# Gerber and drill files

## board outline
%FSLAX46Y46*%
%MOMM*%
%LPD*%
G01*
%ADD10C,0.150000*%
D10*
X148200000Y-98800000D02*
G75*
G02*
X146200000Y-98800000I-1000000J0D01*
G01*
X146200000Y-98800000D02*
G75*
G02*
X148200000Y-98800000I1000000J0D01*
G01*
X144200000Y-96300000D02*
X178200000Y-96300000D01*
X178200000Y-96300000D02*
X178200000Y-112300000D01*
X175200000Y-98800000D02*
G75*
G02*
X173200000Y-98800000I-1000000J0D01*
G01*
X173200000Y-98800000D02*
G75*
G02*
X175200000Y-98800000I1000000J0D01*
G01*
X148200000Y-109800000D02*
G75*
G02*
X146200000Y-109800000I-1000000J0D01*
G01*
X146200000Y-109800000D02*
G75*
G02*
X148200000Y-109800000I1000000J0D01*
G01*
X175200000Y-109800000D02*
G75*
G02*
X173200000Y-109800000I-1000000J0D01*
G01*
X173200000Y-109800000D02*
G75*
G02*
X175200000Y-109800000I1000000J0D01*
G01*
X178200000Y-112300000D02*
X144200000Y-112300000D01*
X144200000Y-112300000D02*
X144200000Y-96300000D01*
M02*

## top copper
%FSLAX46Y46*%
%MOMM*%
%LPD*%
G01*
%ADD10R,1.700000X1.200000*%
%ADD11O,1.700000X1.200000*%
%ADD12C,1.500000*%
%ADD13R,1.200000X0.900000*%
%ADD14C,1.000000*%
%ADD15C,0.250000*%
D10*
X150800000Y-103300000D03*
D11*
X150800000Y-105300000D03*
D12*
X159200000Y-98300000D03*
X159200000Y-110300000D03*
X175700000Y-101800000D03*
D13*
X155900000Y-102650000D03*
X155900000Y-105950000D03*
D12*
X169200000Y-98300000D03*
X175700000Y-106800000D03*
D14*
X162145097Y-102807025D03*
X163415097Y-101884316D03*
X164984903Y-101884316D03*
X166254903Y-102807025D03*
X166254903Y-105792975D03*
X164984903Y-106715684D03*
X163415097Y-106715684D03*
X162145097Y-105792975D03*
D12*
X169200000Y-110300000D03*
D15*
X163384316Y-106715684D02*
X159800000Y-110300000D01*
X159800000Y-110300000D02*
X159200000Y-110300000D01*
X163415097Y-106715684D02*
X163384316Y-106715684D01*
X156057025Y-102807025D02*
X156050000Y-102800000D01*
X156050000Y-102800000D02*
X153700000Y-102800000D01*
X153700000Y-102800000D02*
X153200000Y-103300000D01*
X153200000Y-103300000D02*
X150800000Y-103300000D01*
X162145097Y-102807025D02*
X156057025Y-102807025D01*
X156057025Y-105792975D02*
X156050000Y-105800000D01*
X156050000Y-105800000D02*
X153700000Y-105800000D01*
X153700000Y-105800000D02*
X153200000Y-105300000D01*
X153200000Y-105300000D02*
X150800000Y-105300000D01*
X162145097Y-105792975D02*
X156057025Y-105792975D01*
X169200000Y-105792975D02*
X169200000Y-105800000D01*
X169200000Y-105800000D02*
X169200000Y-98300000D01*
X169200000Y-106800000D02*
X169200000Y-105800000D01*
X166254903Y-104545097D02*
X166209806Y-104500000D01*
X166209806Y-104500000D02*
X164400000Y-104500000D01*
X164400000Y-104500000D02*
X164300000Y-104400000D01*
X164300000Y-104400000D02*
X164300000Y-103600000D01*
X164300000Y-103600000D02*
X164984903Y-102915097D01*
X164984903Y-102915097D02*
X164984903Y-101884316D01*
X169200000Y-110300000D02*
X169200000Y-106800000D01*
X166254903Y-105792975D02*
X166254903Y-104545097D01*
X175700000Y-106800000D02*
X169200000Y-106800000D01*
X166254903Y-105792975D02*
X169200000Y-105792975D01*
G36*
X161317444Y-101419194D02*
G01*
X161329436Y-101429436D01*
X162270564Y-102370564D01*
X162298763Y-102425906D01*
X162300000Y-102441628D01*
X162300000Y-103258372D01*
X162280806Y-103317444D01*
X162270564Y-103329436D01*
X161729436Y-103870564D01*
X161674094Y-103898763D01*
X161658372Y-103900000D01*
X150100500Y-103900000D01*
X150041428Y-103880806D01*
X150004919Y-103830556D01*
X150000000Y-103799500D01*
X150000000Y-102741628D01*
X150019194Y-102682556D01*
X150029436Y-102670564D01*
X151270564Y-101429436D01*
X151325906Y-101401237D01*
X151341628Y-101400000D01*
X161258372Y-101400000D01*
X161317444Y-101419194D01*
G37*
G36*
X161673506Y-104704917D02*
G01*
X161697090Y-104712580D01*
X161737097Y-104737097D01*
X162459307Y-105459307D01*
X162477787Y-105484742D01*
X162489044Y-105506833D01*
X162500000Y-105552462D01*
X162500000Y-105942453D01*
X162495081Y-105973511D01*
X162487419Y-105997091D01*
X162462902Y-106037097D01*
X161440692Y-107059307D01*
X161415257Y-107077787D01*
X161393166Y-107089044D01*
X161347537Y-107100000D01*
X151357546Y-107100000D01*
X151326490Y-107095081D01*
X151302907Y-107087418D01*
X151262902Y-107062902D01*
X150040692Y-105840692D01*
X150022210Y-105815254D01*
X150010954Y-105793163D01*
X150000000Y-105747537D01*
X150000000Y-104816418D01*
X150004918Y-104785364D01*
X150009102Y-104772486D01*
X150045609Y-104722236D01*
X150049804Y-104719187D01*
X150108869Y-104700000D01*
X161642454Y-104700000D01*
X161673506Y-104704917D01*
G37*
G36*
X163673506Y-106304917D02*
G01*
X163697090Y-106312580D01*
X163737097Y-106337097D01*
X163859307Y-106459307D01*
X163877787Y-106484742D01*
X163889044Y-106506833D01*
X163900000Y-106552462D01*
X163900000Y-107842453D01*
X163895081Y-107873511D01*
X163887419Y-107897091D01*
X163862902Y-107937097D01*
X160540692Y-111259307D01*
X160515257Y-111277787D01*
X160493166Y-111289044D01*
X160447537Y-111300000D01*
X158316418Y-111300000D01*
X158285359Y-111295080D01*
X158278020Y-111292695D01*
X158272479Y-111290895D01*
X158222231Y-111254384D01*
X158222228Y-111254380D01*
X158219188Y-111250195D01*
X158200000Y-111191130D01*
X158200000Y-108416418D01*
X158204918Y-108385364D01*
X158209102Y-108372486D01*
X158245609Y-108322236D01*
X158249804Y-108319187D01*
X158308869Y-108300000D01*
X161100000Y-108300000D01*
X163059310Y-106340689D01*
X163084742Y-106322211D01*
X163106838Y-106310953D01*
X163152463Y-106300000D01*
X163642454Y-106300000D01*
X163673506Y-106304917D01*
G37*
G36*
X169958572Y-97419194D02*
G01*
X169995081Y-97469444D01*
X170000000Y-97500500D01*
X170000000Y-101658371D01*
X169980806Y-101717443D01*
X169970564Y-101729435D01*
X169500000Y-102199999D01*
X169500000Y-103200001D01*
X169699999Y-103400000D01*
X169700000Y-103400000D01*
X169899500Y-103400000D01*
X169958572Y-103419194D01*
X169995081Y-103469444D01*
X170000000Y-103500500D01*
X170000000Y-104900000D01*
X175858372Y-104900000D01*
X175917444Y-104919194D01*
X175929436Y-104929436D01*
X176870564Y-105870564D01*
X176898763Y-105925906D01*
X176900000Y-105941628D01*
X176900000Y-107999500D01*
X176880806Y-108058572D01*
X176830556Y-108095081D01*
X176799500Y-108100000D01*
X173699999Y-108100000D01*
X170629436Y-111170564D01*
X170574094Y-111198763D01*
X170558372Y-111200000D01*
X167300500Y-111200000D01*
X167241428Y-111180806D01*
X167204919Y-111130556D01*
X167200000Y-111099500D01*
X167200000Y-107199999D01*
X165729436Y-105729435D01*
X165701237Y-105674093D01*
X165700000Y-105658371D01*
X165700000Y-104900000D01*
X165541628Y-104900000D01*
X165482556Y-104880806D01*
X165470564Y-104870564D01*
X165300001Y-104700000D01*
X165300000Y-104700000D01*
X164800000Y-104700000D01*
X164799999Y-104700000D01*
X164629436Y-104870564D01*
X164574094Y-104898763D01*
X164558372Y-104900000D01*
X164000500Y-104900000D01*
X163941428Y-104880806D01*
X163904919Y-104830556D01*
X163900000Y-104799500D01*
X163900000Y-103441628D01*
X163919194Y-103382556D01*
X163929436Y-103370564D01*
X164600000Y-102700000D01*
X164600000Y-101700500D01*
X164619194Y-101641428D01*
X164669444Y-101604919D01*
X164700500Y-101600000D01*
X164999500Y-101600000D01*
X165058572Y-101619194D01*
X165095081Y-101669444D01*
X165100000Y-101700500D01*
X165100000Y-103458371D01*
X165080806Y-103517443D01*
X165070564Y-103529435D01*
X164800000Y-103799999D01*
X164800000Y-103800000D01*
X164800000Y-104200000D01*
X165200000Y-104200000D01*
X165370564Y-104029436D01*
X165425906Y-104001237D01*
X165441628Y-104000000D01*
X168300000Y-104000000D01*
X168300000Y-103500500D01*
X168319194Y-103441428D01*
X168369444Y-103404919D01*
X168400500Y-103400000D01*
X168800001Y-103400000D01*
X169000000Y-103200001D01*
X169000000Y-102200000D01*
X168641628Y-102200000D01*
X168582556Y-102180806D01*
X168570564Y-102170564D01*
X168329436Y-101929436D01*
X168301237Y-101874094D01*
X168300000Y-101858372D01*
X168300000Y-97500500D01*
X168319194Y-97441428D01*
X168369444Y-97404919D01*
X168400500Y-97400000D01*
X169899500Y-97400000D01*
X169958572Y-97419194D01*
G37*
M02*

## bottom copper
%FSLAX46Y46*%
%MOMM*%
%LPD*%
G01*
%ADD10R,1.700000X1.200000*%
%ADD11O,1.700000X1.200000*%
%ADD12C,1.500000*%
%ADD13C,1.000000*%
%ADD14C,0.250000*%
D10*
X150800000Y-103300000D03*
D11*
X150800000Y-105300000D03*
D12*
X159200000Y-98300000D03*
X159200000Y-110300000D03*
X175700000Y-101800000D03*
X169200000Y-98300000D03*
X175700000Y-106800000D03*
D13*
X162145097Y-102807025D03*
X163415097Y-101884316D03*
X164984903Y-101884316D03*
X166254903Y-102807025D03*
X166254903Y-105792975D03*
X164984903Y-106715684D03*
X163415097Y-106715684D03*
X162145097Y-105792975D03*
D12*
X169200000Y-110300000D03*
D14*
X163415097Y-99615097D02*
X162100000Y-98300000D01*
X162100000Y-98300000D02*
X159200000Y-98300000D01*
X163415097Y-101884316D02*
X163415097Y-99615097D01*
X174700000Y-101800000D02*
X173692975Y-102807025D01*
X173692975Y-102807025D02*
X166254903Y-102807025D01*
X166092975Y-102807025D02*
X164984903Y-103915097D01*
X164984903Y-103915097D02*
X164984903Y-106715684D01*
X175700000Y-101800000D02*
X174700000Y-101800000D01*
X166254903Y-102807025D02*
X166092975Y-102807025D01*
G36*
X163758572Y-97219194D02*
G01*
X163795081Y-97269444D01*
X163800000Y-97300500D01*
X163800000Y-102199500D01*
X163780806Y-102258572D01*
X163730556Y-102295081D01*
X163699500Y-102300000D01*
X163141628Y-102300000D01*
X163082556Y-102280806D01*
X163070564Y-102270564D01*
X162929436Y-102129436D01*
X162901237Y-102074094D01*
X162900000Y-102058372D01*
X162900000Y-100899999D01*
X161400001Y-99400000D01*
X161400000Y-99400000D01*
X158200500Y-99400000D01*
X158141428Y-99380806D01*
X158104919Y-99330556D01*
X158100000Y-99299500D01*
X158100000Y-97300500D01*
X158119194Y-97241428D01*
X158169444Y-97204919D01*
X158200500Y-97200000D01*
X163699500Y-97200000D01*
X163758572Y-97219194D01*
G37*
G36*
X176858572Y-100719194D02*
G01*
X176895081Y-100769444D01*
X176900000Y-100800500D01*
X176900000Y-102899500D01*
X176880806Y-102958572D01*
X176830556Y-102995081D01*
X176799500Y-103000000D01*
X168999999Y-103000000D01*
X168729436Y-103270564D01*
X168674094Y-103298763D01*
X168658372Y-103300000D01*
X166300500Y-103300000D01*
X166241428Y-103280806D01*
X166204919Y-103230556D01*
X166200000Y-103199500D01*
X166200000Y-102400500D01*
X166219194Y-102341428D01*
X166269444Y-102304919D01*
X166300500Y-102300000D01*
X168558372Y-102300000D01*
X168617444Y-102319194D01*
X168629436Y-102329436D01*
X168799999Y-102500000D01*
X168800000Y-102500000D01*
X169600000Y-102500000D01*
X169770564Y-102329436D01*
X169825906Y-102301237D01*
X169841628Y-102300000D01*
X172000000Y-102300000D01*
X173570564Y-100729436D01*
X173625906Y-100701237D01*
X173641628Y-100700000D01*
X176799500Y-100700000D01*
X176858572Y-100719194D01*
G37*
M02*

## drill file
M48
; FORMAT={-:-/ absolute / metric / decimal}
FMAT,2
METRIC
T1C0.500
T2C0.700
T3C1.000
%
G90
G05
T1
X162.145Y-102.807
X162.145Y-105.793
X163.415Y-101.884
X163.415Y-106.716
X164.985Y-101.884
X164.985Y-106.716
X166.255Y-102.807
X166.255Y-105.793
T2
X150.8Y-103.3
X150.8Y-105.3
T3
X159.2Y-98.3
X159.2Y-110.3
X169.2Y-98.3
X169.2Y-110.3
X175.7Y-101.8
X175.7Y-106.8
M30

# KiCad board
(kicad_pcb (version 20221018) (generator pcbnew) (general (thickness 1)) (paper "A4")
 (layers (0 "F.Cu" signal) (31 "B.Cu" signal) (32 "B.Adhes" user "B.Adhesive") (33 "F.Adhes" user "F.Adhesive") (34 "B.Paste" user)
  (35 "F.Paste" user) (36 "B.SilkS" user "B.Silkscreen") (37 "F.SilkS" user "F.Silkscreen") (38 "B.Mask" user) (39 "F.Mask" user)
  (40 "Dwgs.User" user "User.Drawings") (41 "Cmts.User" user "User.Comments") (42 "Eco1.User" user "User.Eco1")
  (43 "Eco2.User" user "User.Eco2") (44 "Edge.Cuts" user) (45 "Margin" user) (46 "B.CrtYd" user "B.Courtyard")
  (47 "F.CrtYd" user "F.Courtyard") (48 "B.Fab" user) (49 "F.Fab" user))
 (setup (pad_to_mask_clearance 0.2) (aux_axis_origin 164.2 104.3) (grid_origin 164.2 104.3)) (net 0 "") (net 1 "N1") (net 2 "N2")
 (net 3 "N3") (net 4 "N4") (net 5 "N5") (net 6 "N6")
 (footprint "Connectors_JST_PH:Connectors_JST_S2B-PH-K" (layer "F.Cu") (at 150.8 103.3 -90)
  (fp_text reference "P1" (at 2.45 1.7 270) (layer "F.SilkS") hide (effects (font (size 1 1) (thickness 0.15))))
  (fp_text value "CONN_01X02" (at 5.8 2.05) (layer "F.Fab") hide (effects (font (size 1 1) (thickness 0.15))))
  (pad "1" thru_hole rect (at 0 0 270) (size 1.2 1.7) (drill 0.7) (layers "*.Cu" "*.Mask" "F.SilkS") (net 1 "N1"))
  (pad "2" thru_hole oval (at 2 0 270) (size 1.2 1.7) (drill 0.7) (layers "*.Cu" "*.Mask" "F.SilkS") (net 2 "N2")))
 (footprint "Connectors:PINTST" (layer "F.Cu") (at 159.2 98.3)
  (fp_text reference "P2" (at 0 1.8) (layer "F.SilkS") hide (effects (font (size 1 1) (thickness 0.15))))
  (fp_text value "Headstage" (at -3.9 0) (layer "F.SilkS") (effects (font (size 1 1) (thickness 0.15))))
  (pad "1" thru_hole circle (at 0 0) (size 1.5 1.5) (drill 1) (layers "*.Cu" "*.Mask") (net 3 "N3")))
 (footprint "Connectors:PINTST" (layer "F.Cu") (at 159.2 110.3)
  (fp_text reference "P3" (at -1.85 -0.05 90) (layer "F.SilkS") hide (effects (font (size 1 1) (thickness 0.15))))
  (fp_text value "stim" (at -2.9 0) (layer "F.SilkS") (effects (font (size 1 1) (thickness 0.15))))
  (pad "1" thru_hole circle (at 0 0) (size 1.5 1.5) (drill 1) (layers "*.Cu" "*.Mask") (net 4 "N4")))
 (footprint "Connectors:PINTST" (layer "F.Cu") (at 175.7 101.8)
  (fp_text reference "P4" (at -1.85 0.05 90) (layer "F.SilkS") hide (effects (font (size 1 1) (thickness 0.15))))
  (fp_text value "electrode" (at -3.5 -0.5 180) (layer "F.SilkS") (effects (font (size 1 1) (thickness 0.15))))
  (pad "1" thru_hole circle (at 0 0) (size 1.5 1.5) (drill 1) (layers "*.Cu" "*.Mask") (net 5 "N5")))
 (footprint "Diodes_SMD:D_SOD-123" (layer "F.Cu") (at 155.9 104.3 -90)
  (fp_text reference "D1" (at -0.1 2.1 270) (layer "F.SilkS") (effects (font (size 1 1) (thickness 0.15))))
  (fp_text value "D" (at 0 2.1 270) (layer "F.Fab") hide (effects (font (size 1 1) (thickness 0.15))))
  (pad "1" smd rect (at -1.65 0 270) (size 0.9 1.2) (layers "F.Cu" "F.Paste" "F.Mask") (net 1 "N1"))
  (pad "2" smd rect (at 1.65 0 270) (size 0.9 1.2) (layers "F.Cu" "F.Paste" "F.Mask") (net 2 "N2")))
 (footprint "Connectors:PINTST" (layer "F.Cu") (at 169.2 98.3)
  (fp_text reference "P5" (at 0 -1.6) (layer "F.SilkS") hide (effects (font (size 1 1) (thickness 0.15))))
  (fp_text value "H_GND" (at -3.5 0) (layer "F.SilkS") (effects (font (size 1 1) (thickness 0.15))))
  (pad "1" thru_hole circle (at 0 0) (size 1.5 1.5) (drill 1) (layers "*.Cu" "*.Mask") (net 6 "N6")))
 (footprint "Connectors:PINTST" (layer "F.Cu") (at 175.7 106.8)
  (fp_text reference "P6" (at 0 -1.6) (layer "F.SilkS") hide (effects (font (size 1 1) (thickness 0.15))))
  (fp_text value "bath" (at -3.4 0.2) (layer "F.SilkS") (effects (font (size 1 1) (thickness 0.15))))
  (pad "1" thru_hole circle (at 0 0) (size 1.5 1.5) (drill 1) (layers "*.Cu" "*.Mask") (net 6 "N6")))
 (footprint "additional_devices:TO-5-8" (layer "F.Cu") (at 164.2 104.3 90)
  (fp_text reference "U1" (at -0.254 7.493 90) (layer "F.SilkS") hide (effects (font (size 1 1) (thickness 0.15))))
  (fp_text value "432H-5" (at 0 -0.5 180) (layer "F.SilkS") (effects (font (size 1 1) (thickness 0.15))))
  (pad "1" thru_hole circle (at 1.492975 -2.054903 90) (size 1 1) (drill 0.5) (layers "*.Cu" "*.Mask") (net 1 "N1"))
  (pad "2" thru_hole circle (at 2.415684 -0.784903 54) (size 1 1) (drill 0.5) (layers "*.Cu" "*.Mask") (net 3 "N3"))
  (pad "3" thru_hole circle (at 2.415684 0.784903 18) (size 1 1) (drill 0.5) (layers "*.Cu" "*.Mask") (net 6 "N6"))
  (pad "4" thru_hole circle (at 1.492975 2.054903 342) (size 1 1) (drill 0.5) (layers "*.Cu" "*.Mask") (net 5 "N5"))
  (pad "5" thru_hole circle (at -1.492975 2.054903 270) (size 1 1) (drill 0.5) (layers "*.Cu" "*.Mask") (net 6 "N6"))
  (pad "6" thru_hole circle (at -2.415684 0.784903 234) (size 1 1) (drill 0.5) (layers "*.Cu" "*.Mask") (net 5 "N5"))
  (pad "7" thru_hole circle (at -2.415684 -0.784903 198) (size 1 1) (drill 0.5) (layers "*.Cu" "*.Mask") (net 4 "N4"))
  (pad "8" thru_hole circle (at -1.492975 -2.054903 162) (size 1 1) (drill 0.5) (layers "*.Cu" "*.Mask") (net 2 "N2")))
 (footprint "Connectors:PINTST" (layer "F.Cu") (at 169.2 110.3)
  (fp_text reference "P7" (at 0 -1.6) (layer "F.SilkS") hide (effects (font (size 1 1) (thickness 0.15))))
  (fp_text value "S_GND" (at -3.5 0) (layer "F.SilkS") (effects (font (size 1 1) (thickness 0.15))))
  (pad "1" thru_hole circle (at 0 0) (size 1.5 1.5) (drill 1) (layers "*.Cu" "*.Mask") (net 6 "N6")))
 (gr_circle (center 147.2 98.8) (end 148.2 98.8) (stroke (width 0.15) (type solid)) (fill none) (layer "Edge.Cuts"))
 (gr_line (start 144.2 96.3) (end 178.2 96.3) (stroke (width 0.15) (type solid)) (layer "Edge.Cuts"))
 (gr_line (start 178.2 96.3) (end 178.2 112.3) (stroke (width 0.15) (type solid)) (layer "Edge.Cuts"))
 (gr_circle (center 174.2 98.8) (end 175.2 98.8) (stroke (width 0.15) (type solid)) (fill none) (layer "Edge.Cuts"))
 (gr_circle (center 147.2 109.8) (end 148.2 109.8) (stroke (width 0.15) (type solid)) (fill none) (layer "Edge.Cuts"))
 (gr_circle (center 174.2 109.8) (end 175.2 109.8) (stroke (width 0.15) (type solid)) (fill none) (layer "Edge.Cuts"))
 (gr_line (start 178.2 112.3) (end 144.2 112.3) (stroke (width 0.15) (type solid)) (layer "Edge.Cuts"))
 (gr_line (start 144.2 112.3) (end 144.2 96.3) (stroke (width 0.15) (type solid)) (layer "Edge.Cuts"))
 (segment (start 163.415097 99.615097) (end 162.1 98.3) (width 0.25) (layer "B.Cu") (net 3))
 (segment (start 162.1 98.3) (end 159.2 98.3) (width 0.25) (layer "B.Cu") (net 3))
 (segment (start 163.415097 101.884316) (end 163.415097 99.615097) (width 0.25) (layer "B.Cu") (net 3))
 (segment (start 163.384316 106.715684) (end 159.8 110.3) (width 0.25) (layer "F.Cu") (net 4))
 (segment (start 159.8 110.3) (end 159.2 110.3) (width 0.25) (layer "F.Cu") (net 4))
 (segment (start 163.415097 106.715684) (end 163.384316 106.715684) (width 0.25) (layer "F.Cu") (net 4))
 (segment (start 174.7 101.8) (end 173.692975 102.807025) (width 0.25) (layer "B.Cu") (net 5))
 (segment (start 173.692975 102.807025) (end 166.254903 102.807025) (width 0.25) (layer "B.Cu") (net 5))
 (segment (start 166.092975 102.807025) (end 164.984903 103.915097) (width 0.25) (layer "B.Cu") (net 5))
 (segment (start 164.984903 103.915097) (end 164.984903 106.715684) (width 0.25) (layer "B.Cu") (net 5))
 (segment (start 175.7 101.8) (end 174.7 101.8) (width 0.25) (layer "B.Cu") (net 5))
 (segment (start 166.254903 102.807025) (end 166.092975 102.807025) (width 0.25) (layer "B.Cu") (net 5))
 (segment (start 156.057025 102.807025) (end 156.05 102.8) (width 0.25) (layer "F.Cu") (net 1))
 (segment (start 156.05 102.8) (end 153.7 102.8) (width 0.25) (layer "F.Cu") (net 1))
 (segment (start 153.7 102.8) (end 153.2 103.3) (width 0.25) (layer "F.Cu") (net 1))
 (segment (start 153.2 103.3) (end 150.8 103.3) (width 0.25) (layer "F.Cu") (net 1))
 (segment (start 162.145097 102.807025) (end 156.057025 102.807025) (width 0.25) (layer "F.Cu") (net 1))
 (segment (start 156.057025 105.792975) (end 156.05 105.8) (width 0.25) (layer "F.Cu") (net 2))
 (segment (start 156.05 105.8) (end 153.7 105.8) (width 0.25) (layer "F.Cu") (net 2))
 (segment (start 153.7 105.8) (end 153.2 105.3) (width 0.25) (layer "F.Cu") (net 2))
 (segment (start 153.2 105.3) (end 150.8 105.3) (width 0.25) (layer "F.Cu") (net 2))
 (segment (start 162.145097 105.792975) (end 156.057025 105.792975) (width 0.25) (layer "F.Cu") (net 2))
 (segment (start 169.2 105.792975) (end 169.2 105.8) (width 0.25) (layer "F.Cu") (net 6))
 (segment (start 169.2 105.8) (end 169.2 98.3) (width 0.25) (layer "F.Cu") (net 6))
 (segment (start 169.2 106.8) (end 169.2 105.8) (width 0.25) (layer "F.Cu") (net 6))
 (segment (start 166.254903 104.545097) (end 166.209806 104.5) (width 0.25) (layer "F.Cu") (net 6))
 (segment (start 166.209806 104.5) (end 164.4 104.5) (width 0.25) (layer "F.Cu") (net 6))
 (segment (start 164.4 104.5) (end 164.3 104.4) (width 0.25) (layer "F.Cu") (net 6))
 (segment (start 164.3 104.4) (end 164.3 103.6) (width 0.25) (layer "F.Cu") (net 6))
 (segment (start 164.3 103.6) (end 164.984903 102.915097) (width 0.25) (layer "F.Cu") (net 6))
 (segment (start 164.984903 102.915097) (end 164.984903 101.884316) (width 0.25) (layer "F.Cu") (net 6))
 (segment (start 169.2 110.3) (end 169.2 106.8) (width 0.25) (layer "F.Cu") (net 6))
 (segment (start 166.254903 105.792975) (end 166.254903 104.545097) (width 0.25) (layer "F.Cu") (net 6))
 (segment (start 175.7 106.8) (end 169.2 106.8) (width 0.25) (layer "F.Cu") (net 6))
 (segment (start 166.254903 105.792975) (end 169.2 105.792975) (width 0.25) (layer "F.Cu") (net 6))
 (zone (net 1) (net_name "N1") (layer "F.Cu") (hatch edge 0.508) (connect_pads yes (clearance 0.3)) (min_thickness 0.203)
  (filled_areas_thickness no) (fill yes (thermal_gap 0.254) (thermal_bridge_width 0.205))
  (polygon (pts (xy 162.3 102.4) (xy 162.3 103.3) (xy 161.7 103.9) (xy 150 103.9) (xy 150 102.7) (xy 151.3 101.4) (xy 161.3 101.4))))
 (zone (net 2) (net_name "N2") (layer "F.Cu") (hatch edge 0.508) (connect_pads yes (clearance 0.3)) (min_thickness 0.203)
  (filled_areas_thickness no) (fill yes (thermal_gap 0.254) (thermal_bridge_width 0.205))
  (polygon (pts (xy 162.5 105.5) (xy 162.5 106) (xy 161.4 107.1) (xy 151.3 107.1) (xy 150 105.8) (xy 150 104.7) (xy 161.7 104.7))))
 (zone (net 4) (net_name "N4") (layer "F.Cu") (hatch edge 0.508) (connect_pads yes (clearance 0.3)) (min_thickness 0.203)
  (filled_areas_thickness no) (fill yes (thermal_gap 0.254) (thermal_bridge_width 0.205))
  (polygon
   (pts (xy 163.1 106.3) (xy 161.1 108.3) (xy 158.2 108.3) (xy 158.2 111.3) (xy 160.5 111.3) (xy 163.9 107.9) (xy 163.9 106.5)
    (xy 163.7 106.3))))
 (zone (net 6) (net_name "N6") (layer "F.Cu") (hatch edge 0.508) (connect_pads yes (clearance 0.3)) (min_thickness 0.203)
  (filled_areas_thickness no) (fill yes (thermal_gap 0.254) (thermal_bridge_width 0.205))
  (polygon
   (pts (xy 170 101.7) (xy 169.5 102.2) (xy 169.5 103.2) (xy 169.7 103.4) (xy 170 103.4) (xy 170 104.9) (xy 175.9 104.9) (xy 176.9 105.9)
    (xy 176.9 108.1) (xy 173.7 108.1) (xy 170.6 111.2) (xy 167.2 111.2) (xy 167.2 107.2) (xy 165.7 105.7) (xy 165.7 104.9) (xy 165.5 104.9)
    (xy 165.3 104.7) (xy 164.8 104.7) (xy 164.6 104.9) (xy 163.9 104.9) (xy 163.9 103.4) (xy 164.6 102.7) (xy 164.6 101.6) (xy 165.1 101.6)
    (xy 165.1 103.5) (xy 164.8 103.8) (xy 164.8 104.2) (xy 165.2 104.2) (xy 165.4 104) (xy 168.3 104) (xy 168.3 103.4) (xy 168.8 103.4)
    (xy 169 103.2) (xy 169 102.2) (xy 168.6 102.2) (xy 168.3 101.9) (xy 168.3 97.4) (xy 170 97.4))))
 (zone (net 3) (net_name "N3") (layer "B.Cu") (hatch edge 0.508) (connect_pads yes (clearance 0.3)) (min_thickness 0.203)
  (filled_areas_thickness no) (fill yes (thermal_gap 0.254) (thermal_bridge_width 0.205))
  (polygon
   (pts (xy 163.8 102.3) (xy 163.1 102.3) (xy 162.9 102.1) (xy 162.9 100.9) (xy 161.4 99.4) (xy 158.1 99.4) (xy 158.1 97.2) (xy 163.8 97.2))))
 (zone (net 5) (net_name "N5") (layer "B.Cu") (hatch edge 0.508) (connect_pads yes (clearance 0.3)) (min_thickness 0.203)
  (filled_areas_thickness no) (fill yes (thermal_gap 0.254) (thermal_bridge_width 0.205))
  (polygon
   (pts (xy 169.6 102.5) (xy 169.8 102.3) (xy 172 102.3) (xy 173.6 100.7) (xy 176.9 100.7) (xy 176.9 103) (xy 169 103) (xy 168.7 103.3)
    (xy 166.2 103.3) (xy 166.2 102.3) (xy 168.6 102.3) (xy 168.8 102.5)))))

